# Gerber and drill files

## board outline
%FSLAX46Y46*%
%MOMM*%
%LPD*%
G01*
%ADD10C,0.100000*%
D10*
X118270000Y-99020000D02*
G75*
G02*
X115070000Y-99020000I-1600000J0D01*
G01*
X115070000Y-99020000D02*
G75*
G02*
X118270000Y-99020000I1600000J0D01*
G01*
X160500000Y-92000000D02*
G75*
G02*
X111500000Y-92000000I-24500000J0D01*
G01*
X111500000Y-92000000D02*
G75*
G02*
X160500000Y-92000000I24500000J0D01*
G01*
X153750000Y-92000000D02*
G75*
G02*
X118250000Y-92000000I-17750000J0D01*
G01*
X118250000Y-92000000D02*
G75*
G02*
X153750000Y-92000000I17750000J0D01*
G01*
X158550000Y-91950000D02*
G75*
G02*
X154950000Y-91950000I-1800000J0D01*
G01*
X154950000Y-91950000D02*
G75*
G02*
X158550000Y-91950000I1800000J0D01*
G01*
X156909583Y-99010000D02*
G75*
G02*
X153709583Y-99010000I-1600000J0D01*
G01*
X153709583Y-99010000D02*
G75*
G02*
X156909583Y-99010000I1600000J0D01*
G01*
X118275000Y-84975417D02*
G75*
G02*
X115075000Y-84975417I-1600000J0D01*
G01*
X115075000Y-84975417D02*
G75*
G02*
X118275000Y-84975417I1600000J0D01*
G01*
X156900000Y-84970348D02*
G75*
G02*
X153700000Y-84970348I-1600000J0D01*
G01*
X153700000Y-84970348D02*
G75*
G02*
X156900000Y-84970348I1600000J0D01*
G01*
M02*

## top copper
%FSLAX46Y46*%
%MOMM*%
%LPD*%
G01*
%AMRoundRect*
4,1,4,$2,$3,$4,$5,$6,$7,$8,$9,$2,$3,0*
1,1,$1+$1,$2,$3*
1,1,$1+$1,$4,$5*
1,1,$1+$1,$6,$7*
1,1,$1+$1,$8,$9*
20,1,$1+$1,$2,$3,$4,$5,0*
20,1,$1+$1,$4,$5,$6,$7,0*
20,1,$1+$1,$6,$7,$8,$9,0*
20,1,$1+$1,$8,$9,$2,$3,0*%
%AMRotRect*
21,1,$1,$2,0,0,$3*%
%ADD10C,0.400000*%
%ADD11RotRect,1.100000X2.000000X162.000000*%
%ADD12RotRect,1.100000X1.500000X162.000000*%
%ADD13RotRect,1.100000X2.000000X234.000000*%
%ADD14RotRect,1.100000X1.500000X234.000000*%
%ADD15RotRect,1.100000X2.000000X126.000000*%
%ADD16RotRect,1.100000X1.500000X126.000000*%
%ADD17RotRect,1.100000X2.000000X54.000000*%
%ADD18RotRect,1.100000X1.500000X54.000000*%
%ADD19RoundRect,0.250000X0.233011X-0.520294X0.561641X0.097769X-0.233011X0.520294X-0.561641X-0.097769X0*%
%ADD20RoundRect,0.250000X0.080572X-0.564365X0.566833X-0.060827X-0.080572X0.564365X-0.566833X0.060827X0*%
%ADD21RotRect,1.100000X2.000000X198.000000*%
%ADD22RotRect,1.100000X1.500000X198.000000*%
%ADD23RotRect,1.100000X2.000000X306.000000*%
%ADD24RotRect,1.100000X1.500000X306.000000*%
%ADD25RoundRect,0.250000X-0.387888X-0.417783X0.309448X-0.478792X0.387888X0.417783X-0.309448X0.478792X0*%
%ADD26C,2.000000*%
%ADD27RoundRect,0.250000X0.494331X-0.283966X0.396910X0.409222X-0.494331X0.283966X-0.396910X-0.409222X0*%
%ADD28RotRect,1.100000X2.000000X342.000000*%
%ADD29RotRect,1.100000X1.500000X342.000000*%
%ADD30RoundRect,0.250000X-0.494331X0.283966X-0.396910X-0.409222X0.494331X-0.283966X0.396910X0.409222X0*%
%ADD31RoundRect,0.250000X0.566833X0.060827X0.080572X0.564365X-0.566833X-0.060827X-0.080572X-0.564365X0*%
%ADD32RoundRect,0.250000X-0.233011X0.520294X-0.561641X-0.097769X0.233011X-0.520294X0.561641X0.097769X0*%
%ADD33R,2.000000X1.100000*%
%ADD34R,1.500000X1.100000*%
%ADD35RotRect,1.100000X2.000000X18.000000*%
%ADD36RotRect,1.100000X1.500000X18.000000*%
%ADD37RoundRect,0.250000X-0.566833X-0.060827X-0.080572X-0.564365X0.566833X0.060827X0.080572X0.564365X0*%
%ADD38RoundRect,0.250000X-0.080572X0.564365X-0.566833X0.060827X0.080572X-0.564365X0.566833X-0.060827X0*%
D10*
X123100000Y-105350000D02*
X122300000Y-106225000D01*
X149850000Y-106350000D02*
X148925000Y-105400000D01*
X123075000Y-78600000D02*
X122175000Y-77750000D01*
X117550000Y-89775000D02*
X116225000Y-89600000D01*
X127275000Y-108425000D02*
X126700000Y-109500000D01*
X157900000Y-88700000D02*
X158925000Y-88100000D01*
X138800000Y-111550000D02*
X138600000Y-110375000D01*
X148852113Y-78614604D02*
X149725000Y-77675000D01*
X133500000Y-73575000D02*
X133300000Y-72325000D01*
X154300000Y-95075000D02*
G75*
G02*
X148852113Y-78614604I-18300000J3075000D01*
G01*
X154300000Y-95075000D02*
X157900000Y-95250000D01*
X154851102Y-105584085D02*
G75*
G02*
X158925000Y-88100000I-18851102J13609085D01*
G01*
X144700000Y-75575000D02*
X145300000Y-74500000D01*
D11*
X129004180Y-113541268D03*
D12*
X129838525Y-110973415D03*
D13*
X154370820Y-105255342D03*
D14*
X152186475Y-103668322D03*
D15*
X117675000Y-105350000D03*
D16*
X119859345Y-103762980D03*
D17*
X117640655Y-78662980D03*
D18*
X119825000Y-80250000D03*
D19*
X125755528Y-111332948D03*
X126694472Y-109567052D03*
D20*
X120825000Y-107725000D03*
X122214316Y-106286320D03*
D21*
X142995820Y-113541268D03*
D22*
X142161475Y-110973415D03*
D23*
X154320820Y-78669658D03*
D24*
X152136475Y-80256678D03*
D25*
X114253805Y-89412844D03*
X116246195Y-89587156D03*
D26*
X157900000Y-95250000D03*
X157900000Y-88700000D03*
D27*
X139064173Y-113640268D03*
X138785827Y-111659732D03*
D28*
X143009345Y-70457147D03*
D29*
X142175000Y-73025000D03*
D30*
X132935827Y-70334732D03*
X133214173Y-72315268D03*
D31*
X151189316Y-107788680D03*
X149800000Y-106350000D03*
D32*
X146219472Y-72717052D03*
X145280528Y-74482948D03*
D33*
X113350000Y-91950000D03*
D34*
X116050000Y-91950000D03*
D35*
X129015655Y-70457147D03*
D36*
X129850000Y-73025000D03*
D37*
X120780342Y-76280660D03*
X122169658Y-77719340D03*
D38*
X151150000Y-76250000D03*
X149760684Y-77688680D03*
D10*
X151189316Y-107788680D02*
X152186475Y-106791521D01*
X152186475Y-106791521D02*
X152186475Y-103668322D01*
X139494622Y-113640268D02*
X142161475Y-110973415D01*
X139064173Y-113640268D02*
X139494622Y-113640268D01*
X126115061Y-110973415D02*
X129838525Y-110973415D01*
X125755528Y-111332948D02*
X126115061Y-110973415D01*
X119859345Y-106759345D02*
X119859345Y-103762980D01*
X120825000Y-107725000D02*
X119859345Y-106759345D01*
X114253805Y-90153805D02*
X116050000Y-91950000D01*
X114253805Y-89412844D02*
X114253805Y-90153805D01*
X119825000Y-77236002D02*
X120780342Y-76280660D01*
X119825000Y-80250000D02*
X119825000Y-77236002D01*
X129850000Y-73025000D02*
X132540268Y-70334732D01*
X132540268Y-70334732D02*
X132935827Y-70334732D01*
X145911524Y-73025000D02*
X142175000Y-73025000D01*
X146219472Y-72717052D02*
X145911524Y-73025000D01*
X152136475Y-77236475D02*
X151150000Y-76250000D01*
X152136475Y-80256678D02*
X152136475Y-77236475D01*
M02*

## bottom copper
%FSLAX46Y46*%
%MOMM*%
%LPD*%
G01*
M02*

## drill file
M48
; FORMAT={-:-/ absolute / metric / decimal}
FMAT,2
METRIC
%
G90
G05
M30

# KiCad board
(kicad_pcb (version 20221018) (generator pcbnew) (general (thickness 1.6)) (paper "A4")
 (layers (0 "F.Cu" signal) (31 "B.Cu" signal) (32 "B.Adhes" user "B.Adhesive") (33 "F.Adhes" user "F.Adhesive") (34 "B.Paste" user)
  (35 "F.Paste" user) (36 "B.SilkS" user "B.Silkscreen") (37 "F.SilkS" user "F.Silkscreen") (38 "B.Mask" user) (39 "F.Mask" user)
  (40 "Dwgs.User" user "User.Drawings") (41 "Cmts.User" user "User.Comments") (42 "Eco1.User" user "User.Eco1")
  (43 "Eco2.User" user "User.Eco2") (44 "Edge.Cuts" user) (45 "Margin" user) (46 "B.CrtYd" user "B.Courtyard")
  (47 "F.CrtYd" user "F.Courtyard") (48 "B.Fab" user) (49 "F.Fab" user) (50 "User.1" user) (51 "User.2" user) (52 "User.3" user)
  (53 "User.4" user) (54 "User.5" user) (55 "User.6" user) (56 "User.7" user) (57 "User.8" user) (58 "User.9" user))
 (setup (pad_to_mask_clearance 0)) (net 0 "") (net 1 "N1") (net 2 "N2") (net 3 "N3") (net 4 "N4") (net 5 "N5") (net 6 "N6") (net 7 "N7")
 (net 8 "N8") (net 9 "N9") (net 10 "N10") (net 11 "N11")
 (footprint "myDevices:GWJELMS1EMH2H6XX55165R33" (layer "F.Cu") (at 129.375 112.4 72)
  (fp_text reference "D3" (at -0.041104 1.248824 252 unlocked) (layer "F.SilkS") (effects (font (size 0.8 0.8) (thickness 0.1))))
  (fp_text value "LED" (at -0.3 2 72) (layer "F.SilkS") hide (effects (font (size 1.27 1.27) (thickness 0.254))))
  (pad "1" smd rect (at -1.2 0 162) (size 1.1 2) (layers "F.Cu" "F.Paste" "F.Mask") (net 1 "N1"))
  (pad "2" smd rect (at 1.5 0 162) (size 1.1 1.5) (layers "F.Cu" "F.Paste" "F.Mask") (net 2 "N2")))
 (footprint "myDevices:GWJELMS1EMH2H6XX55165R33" (layer "F.Cu") (at 153.4 104.55 144)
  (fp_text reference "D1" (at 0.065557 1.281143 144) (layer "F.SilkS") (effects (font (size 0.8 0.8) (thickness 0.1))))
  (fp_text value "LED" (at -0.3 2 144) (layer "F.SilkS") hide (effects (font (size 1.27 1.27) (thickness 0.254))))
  (pad "1" smd rect (at -1.2 0 234) (size 1.1 2) (layers "F.Cu" "F.Paste" "F.Mask") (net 1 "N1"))
  (pad "2" smd rect (at 1.5 0 234) (size 1.1 1.5) (layers "F.Cu" "F.Paste" "F.Mask") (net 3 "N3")))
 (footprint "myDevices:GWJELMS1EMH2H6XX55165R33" (layer "F.Cu") (at 118.64582 104.644658 36)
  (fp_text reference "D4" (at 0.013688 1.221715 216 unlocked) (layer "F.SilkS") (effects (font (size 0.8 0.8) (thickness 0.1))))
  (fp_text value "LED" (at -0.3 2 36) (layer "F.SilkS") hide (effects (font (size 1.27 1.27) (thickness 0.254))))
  (pad "1" smd rect (at -1.2 0 126) (size 1.1 2) (layers "F.Cu" "F.Paste" "F.Mask") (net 1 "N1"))
  (pad "2" smd rect (at 1.5 0 126) (size 1.1 1.5) (layers "F.Cu" "F.Paste" "F.Mask") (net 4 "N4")))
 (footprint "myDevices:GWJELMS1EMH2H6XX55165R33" (layer "F.Cu") (at 118.611475 79.368322 -36)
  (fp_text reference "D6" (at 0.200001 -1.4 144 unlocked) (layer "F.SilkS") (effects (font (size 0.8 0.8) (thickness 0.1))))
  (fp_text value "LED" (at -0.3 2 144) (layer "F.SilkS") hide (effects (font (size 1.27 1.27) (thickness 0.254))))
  (pad "1" smd rect (at -1.2 0 54) (size 1.1 2) (layers "F.Cu" "F.Paste" "F.Mask") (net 1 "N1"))
  (pad "2" smd rect (at 1.5 0 54) (size 1.1 1.5) (layers "F.Cu" "F.Paste" "F.Mask") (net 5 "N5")))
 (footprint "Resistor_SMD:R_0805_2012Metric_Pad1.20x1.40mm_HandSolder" (layer "F.Cu") (at 126.225 110.45 62)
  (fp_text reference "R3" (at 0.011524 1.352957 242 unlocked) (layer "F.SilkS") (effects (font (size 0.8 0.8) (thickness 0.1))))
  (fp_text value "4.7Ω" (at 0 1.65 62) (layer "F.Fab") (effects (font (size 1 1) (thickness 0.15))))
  (pad "1" smd roundrect (at -1 0 62) (size 1.2 1.4) (layers "F.Cu" "F.Paste" "F.Mask") (roundrect_rratio 0.2083333333) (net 2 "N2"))
  (pad "2" smd roundrect (at 1 0 62) (size 1.2 1.4) (layers "F.Cu" "F.Paste" "F.Mask") (roundrect_rratio 0.2083333333) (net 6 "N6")))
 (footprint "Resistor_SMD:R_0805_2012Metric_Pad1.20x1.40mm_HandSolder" (layer "F.Cu") (at 121.519658 107.00566 46)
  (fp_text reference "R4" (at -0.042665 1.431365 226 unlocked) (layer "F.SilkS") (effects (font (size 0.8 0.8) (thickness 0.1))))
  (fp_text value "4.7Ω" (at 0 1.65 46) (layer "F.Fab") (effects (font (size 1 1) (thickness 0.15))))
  (pad "1" smd roundrect (at -1 0 46) (size 1.2 1.4) (layers "F.Cu" "F.Paste" "F.Mask") (roundrect_rratio 0.2083333333) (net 4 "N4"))
  (pad "2" smd roundrect (at 1 0 46) (size 1.2 1.4) (layers "F.Cu" "F.Paste" "F.Mask") (roundrect_rratio 0.2083333333) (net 6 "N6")))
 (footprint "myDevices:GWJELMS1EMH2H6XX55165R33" (layer "F.Cu") (at 142.625 112.4 108)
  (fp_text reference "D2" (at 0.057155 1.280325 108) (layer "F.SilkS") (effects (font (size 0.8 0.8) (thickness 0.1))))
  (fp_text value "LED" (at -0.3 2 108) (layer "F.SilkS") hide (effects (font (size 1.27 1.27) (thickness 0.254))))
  (pad "1" smd rect (at -1.2 0 198) (size 1.1 2) (layers "F.Cu" "F.Paste" "F.Mask") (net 1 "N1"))
  (pad "2" smd rect (at 1.5 0 198) (size 1.1 1.5) (layers "F.Cu" "F.Paste" "F.Mask") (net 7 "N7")))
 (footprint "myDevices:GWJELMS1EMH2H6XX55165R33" (layer "F.Cu") (at 153.35 79.375 -144)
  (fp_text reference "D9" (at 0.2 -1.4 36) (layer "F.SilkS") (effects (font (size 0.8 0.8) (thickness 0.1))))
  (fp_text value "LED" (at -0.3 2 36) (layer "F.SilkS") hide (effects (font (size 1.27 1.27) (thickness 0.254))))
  (pad "1" smd rect (at -1.2 0 306) (size 1.1 2) (layers "F.Cu" "F.Paste" "F.Mask") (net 1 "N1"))
  (pad "2" smd rect (at 1.5 0 306) (size 1.1 1.5) (layers "F.Cu" "F.Paste" "F.Mask") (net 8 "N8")))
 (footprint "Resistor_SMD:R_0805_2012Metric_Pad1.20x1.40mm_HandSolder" (layer "F.Cu") (at 115.25 89.5 -5)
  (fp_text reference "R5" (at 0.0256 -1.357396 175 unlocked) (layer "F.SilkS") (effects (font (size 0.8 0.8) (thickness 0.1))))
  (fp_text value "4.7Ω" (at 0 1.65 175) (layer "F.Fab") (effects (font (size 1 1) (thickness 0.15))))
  (pad "1" smd roundrect (at -1 0 355) (size 1.2 1.4) (layers "F.Cu" "F.Paste" "F.Mask") (roundrect_rratio 0.2083333333) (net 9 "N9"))
  (pad "2" smd roundrect (at 1 0 355) (size 1.2 1.4) (layers "F.Cu" "F.Paste" "F.Mask") (roundrect_rratio 0.2083333333) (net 6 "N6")))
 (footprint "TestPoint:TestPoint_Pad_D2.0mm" (layer "F.Cu") (at 157.9 95.25)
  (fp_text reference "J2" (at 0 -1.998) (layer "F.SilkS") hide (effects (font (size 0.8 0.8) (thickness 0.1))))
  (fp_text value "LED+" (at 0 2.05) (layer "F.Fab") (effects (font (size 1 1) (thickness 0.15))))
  (pad "1" smd circle (at 0 0) (size 2 2) (layers "F.Cu" "F.Mask") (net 6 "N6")))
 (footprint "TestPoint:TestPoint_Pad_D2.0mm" (layer "F.Cu") (at 157.9 88.7)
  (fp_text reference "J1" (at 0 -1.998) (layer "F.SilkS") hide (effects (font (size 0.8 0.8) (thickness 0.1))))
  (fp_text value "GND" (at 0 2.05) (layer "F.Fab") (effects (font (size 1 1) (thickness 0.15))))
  (pad "1" smd circle (at 0 0) (size 2 2) (layers "F.Cu" "F.Mask") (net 1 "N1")))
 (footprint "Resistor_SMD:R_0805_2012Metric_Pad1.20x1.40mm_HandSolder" (layer "F.Cu") (at 138.925 112.65 98)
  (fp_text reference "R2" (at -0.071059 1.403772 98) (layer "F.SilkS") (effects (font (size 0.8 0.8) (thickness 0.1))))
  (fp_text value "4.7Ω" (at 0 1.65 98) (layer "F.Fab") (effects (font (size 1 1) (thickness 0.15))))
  (pad "1" smd roundrect (at -1 0 98) (size 1.2 1.4) (layers "F.Cu" "F.Paste" "F.Mask") (roundrect_rratio 0.2083333333) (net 7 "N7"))
  (pad "2" smd roundrect (at 1 0 98) (size 1.2 1.4) (layers "F.Cu" "F.Paste" "F.Mask") (roundrect_rratio 0.2083333333) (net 6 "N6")))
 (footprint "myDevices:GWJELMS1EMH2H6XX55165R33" (layer "F.Cu") (at 142.638525 71.598415 -108)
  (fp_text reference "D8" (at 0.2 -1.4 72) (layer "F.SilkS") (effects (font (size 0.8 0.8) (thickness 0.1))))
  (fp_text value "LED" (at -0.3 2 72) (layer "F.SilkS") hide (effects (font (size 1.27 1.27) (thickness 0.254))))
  (pad "1" smd rect (at -1.2 0 342) (size 1.1 2) (layers "F.Cu" "F.Paste" "F.Mask") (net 1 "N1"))
  (pad "2" smd rect (at 1.5 0 342) (size 1.1 1.5) (layers "F.Cu" "F.Paste" "F.Mask") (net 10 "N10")))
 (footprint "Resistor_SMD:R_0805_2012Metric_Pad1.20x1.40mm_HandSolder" (layer "F.Cu") (at 133.075 71.325 -82)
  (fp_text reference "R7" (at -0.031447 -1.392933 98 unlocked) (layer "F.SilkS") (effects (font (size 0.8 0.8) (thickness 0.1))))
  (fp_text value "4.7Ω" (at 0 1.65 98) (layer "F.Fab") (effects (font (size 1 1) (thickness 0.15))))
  (pad "1" smd roundrect (at -1 0 278) (size 1.2 1.4) (layers "F.Cu" "F.Paste" "F.Mask") (roundrect_rratio 0.2083333333) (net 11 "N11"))
  (pad "2" smd roundrect (at 1 0 278) (size 1.2 1.4) (layers "F.Cu" "F.Paste" "F.Mask") (roundrect_rratio 0.2083333333) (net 6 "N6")))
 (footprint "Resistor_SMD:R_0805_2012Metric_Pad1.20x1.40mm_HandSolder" (layer "F.Cu") (at 150.494658 107.06934 134)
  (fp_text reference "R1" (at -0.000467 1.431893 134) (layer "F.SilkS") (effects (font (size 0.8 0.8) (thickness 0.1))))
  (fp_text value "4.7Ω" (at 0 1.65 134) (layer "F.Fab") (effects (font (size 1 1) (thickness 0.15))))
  (pad "1" smd roundrect (at -1 0 134) (size 1.2 1.4) (layers "F.Cu" "F.Paste" "F.Mask") (roundrect_rratio 0.2083333333) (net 3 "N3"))
  (pad "2" smd roundrect (at 1 0 134) (size 1.2 1.4) (layers "F.Cu" "F.Paste" "F.Mask") (roundrect_rratio 0.2083333333) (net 6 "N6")))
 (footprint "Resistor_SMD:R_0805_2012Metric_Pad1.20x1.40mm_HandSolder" (layer "F.Cu") (at 145.75 73.6 -118)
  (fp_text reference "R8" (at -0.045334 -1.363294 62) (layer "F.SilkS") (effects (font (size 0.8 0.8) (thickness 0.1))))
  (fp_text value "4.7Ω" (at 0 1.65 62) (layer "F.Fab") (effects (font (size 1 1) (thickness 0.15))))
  (pad "1" smd roundrect (at -1 0 242) (size 1.2 1.4) (layers "F.Cu" "F.Paste" "F.Mask") (roundrect_rratio 0.2083333333) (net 10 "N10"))
  (pad "2" smd roundrect (at 1 0 242) (size 1.2 1.4) (layers "F.Cu" "F.Paste" "F.Mask") (roundrect_rratio 0.2083333333) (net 6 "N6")))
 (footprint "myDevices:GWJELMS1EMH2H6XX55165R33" (layer "F.Cu") (at 114.55 91.95)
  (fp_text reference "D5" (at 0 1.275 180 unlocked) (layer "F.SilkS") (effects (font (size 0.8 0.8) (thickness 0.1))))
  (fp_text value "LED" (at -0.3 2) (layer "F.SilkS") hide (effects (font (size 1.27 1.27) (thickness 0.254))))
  (pad "1" smd rect (at -1.2 0 90) (size 1.1 2) (layers "F.Cu" "F.Paste" "F.Mask") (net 1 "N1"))
  (pad "2" smd rect (at 1.5 0 90) (size 1.1 1.5) (layers "F.Cu" "F.Paste" "F.Mask") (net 9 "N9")))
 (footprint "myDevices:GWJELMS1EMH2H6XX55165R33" (layer "F.Cu") (at 129.386475 71.598415 -72)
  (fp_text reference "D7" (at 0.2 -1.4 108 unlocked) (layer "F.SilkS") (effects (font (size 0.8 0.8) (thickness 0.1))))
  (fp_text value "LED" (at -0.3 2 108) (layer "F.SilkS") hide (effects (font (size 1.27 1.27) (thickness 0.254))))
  (pad "1" smd rect (at -1.2 0 18) (size 1.1 2) (layers "F.Cu" "F.Paste" "F.Mask") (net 1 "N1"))
  (pad "2" smd rect (at 1.5 0 18) (size 1.1 1.5) (layers "F.Cu" "F.Paste" "F.Mask") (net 11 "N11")))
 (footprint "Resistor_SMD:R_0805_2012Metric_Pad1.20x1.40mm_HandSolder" (layer "F.Cu") (at 121.475 77 -46)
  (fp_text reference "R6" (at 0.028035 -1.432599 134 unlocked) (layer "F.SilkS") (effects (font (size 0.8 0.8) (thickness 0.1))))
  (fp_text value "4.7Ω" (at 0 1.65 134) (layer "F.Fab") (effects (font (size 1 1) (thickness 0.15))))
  (pad "1" smd roundrect (at -1 0 314) (size 1.2 1.4) (layers "F.Cu" "F.Paste" "F.Mask") (roundrect_rratio 0.2083333333) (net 5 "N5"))
  (pad "2" smd roundrect (at 1 0 314) (size 1.2 1.4) (layers "F.Cu" "F.Paste" "F.Mask") (roundrect_rratio 0.2083333333) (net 6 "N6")))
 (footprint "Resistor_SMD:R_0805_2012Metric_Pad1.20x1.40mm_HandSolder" (layer "F.Cu") (at 150.455342 76.96934 -134)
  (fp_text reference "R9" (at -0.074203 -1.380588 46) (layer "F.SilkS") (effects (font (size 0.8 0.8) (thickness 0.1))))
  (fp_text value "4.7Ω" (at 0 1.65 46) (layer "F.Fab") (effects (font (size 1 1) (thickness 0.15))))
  (pad "1" smd roundrect (at -1 0 226) (size 1.2 1.4) (layers "F.Cu" "F.Paste" "F.Mask") (roundrect_rratio 0.2083333333) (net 8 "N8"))
  (pad "2" smd roundrect (at 1 0 226) (size 1.2 1.4) (layers "F.Cu" "F.Paste" "F.Mask") (roundrect_rratio 0.2083333333) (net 6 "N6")))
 (gr_line (start 123.1 105.35) (end 122.3 106.225) (stroke (width 0.4) (type default)) (layer "F.Cu"))
 (gr_line (start 149.85 106.35) (end 148.925 105.4) (stroke (width 0.4) (type default)) (layer "F.Cu"))
 (gr_line (start 123.075 78.6) (end 122.175 77.75) (stroke (width 0.4) (type default)) (layer "F.Cu"))
 (gr_line (start 117.55 89.775) (end 116.225 89.6) (stroke (width 0.4) (type default)) (layer "F.Cu"))
 (gr_line (start 127.275 108.425) (end 126.7 109.5) (stroke (width 0.4) (type default)) (layer "F.Cu"))
 (gr_line (start 157.9 88.7) (end 158.925 88.1) (stroke (width 0.4) (type default)) (layer "F.Cu"))
 (gr_line (start 138.8 111.55) (end 138.6 110.375) (stroke (width 0.4) (type default)) (layer "F.Cu"))
 (gr_line (start 148.852113 78.614604) (end 149.725 77.675) (stroke (width 0.4) (type default)) (layer "F.Cu"))
 (gr_line (start 133.5 73.575) (end 133.3 72.325) (stroke (width 0.4) (type default)) (layer "F.Cu"))
 (gr_arc (start 154.3 95.075) (mid 118.383255 97.830601) (end 148.852113 78.614604) (stroke (width 0.4) (type default)) (layer "F.Cu"))
 (gr_line (start 154.3 95.075) (end 157.9 95.25) (stroke (width 0.4) (type default)) (layer "F.Cu"))
 (gr_arc (start 154.851102 105.584085) (mid 113.356372 86.698897) (end 158.925 88.1) (stroke (width 0.4) (type default)) (layer "F.Cu"))
 (gr_line (start 144.7 75.575) (end 145.3 74.5) (stroke (width 0.4) (type default)) (layer "F.Cu"))
 (gr_circle (center 116.67 99.02) (end 118.27 99.02) (stroke (width 0.1) (type default)) (fill none) (layer "Edge.Cuts"))
 (gr_circle (center 136 92) (end 160.5 92) (stroke (width 0.1) (type default)) (fill none) (layer "Edge.Cuts"))
 (gr_circle (center 136 92) (end 153.75 92) (stroke (width 0.1) (type default)) (fill none) (layer "Edge.Cuts"))
 (gr_circle (center 156.75 91.95) (end 158.55 91.95) (stroke (width 0.1) (type default)) (fill none) (layer "Edge.Cuts"))
 (gr_circle (center 155.309583 99.01) (end 156.909583 99.01) (stroke (width 0.1) (type default)) (fill none) (layer "Edge.Cuts"))
 (gr_circle (center 116.675 84.975417) (end 118.275 84.975417) (stroke (width 0.1) (type default)) (fill none) (layer "Edge.Cuts"))
 (gr_circle (center 155.3 84.970348) (end 156.9 84.970348) (stroke (width 0.1) (type default)) (fill none) (layer "Edge.Cuts"))
 (segment (start 151.189316 107.78868) (end 152.186475 106.791521) (width 0.4) (layer "F.Cu") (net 3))
 (segment (start 152.186475 106.791521) (end 152.186475 103.668322) (width 0.4) (layer "F.Cu") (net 3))
 (segment (start 139.494622 113.640268) (end 142.161475 110.973415) (width 0.4) (layer "F.Cu") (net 7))
 (segment (start 139.064173 113.640268) (end 139.494622 113.640268) (width 0.4) (layer "F.Cu") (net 7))
 (segment (start 126.115061 110.973415) (end 129.838525 110.973415) (width 0.4) (layer "F.Cu") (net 2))
 (segment (start 125.755528 111.332948) (end 126.115061 110.973415) (width 0.4) (layer "F.Cu") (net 2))
 (segment (start 119.859345 106.759345) (end 119.859345 103.76298) (width 0.4) (layer "F.Cu") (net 4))
 (segment (start 120.825 107.725) (end 119.859345 106.759345) (width 0.4) (layer "F.Cu") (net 4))
 (segment (start 114.253805 90.153805) (end 116.05 91.95) (width 0.4) (layer "F.Cu") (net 9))
 (segment (start 114.253805 89.412844) (end 114.253805 90.153805) (width 0.4) (layer "F.Cu") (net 9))
 (segment (start 119.825 77.236002) (end 120.780342 76.28066) (width 0.4) (layer "F.Cu") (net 5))
 (segment (start 119.825 80.25) (end 119.825 77.236002) (width 0.4) (layer "F.Cu") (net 5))
 (segment (start 129.85 73.025) (end 132.540268 70.334732) (width 0.4) (layer "F.Cu") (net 11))
 (segment (start 132.540268 70.334732) (end 132.935827 70.334732) (width 0.4) (layer "F.Cu") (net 11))
 (segment (start 145.911524 73.025) (end 142.175 73.025) (width 0.4) (layer "F.Cu") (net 10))
 (segment (start 146.219472 72.717052) (end 145.911524 73.025) (width 0.4) (layer "F.Cu") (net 10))
 (segment (start 152.136475 77.236475) (end 151.15 76.25) (width 0.4) (layer "F.Cu") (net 8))
 (segment (start 152.136475 80.256678) (end 152.136475 77.236475) (width 0.4) (layer "F.Cu") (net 8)))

